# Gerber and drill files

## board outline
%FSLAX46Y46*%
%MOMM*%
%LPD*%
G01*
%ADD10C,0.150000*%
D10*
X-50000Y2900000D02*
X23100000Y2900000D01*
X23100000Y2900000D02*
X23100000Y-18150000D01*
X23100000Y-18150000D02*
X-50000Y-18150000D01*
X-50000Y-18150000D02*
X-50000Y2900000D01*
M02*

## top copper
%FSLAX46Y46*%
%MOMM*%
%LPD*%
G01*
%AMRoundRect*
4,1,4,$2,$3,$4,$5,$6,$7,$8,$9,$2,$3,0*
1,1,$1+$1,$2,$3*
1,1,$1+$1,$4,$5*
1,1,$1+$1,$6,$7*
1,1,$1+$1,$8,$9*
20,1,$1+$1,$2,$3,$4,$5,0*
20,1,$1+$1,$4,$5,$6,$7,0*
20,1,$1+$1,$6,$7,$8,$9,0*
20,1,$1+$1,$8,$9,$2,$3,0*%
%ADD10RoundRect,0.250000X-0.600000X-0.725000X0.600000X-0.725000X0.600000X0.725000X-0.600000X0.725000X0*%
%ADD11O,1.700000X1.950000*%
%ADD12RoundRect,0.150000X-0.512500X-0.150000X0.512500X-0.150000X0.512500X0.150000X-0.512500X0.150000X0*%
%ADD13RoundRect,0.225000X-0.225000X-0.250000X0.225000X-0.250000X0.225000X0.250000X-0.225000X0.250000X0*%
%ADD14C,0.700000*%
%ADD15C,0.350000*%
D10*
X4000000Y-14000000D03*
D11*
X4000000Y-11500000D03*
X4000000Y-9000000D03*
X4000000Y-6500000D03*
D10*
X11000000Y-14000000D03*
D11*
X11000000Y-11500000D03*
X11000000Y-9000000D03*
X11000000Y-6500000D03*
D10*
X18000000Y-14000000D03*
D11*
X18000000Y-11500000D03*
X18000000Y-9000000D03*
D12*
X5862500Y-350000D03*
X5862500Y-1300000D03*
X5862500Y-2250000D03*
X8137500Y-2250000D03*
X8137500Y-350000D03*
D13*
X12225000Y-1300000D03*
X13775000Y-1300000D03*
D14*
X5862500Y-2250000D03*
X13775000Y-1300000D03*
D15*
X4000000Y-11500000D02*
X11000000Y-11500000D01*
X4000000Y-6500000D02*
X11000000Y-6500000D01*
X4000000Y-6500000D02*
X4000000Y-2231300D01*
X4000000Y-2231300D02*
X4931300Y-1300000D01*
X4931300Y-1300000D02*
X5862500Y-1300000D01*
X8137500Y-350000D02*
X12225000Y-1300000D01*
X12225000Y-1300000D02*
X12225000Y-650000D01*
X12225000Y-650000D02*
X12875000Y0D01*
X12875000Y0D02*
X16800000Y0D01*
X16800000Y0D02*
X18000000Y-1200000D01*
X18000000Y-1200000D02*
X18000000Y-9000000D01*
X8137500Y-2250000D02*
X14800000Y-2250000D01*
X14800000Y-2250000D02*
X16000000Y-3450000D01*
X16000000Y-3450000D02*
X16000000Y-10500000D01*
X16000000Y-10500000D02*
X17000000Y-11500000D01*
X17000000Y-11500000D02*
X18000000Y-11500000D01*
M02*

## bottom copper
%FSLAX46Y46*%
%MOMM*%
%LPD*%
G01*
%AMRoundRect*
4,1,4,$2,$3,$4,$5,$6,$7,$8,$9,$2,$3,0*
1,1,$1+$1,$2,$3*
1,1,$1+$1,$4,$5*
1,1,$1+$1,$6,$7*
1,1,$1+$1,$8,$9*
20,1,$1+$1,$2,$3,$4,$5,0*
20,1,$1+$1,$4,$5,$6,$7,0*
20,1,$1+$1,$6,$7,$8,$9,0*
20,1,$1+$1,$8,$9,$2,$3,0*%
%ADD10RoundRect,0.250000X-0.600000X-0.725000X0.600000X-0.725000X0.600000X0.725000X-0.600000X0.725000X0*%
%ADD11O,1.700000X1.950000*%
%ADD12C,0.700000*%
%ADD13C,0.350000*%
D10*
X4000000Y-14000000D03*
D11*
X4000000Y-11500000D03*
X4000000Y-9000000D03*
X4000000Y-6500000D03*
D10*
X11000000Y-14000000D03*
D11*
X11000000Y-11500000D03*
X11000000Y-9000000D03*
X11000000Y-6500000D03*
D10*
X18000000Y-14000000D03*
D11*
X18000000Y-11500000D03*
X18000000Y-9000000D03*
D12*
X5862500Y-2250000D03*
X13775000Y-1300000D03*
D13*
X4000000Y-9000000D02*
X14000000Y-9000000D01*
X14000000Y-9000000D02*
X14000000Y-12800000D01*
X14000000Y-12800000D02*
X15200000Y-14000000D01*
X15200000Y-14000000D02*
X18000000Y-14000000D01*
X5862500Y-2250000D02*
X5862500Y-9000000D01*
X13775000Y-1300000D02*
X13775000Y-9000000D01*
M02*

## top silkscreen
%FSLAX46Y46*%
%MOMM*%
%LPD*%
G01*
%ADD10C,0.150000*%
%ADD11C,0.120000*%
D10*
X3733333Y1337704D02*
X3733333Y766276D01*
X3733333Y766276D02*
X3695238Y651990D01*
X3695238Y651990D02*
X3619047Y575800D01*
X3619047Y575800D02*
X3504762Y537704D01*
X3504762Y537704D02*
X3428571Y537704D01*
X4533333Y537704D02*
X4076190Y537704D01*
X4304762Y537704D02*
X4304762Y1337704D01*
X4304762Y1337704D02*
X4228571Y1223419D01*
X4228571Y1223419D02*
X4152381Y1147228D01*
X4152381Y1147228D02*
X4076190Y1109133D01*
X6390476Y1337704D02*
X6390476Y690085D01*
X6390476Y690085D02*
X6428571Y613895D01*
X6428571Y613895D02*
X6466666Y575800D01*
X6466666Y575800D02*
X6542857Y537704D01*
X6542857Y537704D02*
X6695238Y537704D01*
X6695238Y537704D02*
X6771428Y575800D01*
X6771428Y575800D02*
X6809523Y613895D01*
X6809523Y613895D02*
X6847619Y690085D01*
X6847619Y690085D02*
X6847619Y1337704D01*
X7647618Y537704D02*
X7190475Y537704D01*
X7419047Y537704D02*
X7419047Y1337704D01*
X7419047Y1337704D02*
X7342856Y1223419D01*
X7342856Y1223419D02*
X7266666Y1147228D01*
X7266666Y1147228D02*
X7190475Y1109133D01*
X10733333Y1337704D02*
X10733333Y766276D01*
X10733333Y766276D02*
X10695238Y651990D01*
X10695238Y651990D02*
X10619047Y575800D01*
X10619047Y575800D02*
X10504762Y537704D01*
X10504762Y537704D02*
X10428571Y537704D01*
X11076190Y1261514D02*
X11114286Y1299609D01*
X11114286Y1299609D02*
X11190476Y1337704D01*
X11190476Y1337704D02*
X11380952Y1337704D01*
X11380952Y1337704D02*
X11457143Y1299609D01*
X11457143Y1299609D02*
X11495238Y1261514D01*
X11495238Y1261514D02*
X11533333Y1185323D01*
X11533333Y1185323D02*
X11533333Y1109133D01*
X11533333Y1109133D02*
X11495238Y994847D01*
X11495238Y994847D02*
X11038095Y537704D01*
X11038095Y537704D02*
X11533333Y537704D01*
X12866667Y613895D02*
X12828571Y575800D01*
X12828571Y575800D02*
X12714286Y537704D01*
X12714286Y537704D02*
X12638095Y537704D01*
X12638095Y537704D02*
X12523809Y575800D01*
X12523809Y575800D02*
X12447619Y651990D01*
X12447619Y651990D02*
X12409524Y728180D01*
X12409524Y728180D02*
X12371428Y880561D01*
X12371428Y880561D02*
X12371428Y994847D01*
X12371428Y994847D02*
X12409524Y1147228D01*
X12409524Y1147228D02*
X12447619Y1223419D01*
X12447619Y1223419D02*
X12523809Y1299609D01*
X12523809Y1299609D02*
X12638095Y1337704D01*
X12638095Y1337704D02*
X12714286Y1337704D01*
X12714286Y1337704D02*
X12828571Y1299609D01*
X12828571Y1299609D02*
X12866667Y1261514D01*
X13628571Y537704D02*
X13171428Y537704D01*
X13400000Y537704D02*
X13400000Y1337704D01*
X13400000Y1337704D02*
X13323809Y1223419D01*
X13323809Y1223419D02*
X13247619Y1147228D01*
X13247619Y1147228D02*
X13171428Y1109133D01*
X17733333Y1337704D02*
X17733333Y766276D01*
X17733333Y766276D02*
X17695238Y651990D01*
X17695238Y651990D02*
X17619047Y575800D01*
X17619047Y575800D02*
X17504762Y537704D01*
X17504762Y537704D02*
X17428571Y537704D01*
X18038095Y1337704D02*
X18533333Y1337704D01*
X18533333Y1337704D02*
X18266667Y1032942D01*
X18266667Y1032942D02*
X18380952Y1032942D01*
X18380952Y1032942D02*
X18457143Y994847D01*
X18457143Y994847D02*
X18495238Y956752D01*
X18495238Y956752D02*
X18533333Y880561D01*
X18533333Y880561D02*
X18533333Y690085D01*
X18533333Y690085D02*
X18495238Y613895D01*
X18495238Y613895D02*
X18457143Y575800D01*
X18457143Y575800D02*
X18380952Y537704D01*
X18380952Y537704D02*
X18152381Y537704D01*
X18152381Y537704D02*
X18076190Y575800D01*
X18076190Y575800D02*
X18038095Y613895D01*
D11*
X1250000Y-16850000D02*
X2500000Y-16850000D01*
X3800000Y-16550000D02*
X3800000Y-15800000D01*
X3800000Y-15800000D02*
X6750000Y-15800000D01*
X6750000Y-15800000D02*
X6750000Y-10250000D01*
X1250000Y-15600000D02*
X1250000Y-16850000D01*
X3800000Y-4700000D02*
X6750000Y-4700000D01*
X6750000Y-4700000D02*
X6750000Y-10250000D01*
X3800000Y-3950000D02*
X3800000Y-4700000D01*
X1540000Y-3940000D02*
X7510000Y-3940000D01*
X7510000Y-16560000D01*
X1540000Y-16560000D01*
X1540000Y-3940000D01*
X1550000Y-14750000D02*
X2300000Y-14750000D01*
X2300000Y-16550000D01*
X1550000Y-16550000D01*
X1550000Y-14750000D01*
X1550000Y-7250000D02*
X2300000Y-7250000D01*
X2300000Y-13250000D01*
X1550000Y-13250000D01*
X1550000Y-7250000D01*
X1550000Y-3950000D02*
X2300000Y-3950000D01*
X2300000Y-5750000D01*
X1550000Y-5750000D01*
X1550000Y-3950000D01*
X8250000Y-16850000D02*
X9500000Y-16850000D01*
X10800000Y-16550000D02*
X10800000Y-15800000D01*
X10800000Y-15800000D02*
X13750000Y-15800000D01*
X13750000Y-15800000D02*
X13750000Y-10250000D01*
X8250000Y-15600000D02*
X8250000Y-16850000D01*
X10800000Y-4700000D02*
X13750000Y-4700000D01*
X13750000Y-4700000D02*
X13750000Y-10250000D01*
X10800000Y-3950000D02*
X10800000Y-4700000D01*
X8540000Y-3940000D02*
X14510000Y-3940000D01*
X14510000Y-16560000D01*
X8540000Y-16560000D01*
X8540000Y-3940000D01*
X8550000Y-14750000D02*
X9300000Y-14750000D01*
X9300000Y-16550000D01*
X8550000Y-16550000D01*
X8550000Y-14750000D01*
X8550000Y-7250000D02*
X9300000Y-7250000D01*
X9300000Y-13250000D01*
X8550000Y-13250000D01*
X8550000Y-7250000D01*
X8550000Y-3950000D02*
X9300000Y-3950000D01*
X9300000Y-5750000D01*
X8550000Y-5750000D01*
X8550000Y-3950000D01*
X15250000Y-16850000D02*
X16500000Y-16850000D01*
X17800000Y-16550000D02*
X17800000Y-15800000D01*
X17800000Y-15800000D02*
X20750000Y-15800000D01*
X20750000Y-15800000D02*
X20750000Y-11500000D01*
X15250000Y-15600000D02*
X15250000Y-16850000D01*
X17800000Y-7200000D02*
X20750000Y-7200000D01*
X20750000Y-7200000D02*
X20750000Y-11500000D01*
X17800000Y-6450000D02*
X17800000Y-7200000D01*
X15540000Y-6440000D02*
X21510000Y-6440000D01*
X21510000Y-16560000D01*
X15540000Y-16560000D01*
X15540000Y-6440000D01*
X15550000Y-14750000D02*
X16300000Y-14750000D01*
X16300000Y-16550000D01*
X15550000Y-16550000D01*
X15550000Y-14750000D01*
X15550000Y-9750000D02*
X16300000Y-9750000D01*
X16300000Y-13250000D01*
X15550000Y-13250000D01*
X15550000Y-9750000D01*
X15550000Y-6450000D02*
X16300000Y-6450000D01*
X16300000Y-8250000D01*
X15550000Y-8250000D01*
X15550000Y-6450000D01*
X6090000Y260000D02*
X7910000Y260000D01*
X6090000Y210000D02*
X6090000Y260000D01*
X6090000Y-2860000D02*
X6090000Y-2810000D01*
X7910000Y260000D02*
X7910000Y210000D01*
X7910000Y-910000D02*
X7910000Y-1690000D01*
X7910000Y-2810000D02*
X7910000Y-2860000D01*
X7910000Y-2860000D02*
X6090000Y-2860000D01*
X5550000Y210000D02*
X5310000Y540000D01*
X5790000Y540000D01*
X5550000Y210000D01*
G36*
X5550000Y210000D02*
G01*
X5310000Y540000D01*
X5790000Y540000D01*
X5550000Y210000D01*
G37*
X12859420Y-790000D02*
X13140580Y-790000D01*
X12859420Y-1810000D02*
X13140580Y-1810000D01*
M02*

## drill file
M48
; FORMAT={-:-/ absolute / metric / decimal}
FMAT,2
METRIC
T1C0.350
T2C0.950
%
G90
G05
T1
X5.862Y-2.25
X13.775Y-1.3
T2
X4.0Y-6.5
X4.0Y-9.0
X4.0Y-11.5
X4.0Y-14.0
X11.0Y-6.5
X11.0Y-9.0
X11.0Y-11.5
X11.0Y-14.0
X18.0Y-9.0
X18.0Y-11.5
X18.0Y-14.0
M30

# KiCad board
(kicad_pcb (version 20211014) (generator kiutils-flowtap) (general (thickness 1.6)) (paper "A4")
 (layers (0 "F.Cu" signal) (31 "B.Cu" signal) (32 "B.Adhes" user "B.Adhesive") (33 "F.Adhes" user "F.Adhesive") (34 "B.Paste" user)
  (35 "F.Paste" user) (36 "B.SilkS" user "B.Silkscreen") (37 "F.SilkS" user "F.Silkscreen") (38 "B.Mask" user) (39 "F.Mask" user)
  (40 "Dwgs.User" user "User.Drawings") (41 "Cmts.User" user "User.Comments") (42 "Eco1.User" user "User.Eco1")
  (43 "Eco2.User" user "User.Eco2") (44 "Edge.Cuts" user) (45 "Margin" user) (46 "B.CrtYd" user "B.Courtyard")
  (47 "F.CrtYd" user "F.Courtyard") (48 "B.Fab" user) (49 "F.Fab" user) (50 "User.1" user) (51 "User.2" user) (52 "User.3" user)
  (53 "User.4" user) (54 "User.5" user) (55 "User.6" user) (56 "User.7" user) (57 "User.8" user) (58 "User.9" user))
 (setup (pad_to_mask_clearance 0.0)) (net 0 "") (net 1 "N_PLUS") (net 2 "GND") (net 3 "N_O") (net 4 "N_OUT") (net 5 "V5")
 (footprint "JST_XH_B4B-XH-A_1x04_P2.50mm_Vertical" (layer "F.Cu") (at 4 14 90) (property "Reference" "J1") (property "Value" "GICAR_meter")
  (fp_line (start -2.85 -2.75) (end -2.85 -1.5) (layer "F.SilkS") (stroke (width 0.12) (type solid)))
  (fp_line (start -2.55 -0.2) (end -1.8 -0.2) (layer "F.SilkS") (stroke (width 0.12) (type solid)))
  (fp_line (start -1.8 -0.2) (end -1.8 2.75) (layer "F.SilkS") (stroke (width 0.12) (type solid)))
  (fp_line (start -1.8 2.75) (end 3.75 2.75) (layer "F.SilkS") (stroke (width 0.12) (type solid)))
  (fp_line (start -1.6 -2.75) (end -2.85 -2.75) (layer "F.SilkS") (stroke (width 0.12) (type solid)))
  (fp_line (start 9.3 -0.2) (end 9.3 2.75) (layer "F.SilkS") (stroke (width 0.12) (type solid)))
  (fp_line (start 9.3 2.75) (end 3.75 2.75) (layer "F.SilkS") (stroke (width 0.12) (type solid)))
  (fp_line (start 10.05 -0.2) (end 9.3 -0.2) (layer "F.SilkS") (stroke (width 0.12) (type solid)))
  (fp_rect (start -2.56 -2.46) (end 10.06 3.51) (layer "F.SilkS") (stroke (width 0.12) (type solid)) (fill no))
  (fp_rect (start -2.55 -2.45) (end -0.75 -1.7) (layer "F.SilkS") (stroke (width 0.12) (type solid)) (fill no))
  (fp_rect (start 0.75 -2.45) (end 6.75 -1.7) (layer "F.SilkS") (stroke (width 0.12) (type solid)) (fill no))
  (fp_rect (start 8.25 -2.45) (end 10.05 -1.7) (layer "F.SilkS") (stroke (width 0.12) (type solid)) (fill no))
  (pad "1" thru_hole roundrect (at 0 0) (size 1.7 1.95) (drill 0.95) (layers *.Cu *.Mask) (remove_unused_layers no)
   (roundrect_rratio 0.147059))
  (pad "2" thru_hole oval (at 2.5 0) (size 1.7 1.95) (drill 0.95) (layers *.Cu *.Mask) (remove_unused_layers no) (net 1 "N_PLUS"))
  (pad "3" thru_hole oval (at 5 0) (size 1.7 1.95) (drill 0.95) (layers *.Cu *.Mask) (remove_unused_layers no) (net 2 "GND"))
  (pad "4" thru_hole oval (at 7.5 0) (size 1.7 1.95) (drill 0.95) (layers *.Cu *.Mask) (remove_unused_layers no) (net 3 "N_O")))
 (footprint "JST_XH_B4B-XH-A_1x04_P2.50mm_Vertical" (layer "F.Cu") (at 11 14 90) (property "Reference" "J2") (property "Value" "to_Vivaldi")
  (fp_line (start -2.85 -2.75) (end -2.85 -1.5) (layer "F.SilkS") (stroke (width 0.12) (type solid)))
  (fp_line (start -2.55 -0.2) (end -1.8 -0.2) (layer "F.SilkS") (stroke (width 0.12) (type solid)))
  (fp_line (start -1.8 -0.2) (end -1.8 2.75) (layer "F.SilkS") (stroke (width 0.12) (type solid)))
  (fp_line (start -1.8 2.75) (end 3.75 2.75) (layer "F.SilkS") (stroke (width 0.12) (type solid)))
  (fp_line (start -1.6 -2.75) (end -2.85 -2.75) (layer "F.SilkS") (stroke (width 0.12) (type solid)))
  (fp_line (start 9.3 -0.2) (end 9.3 2.75) (layer "F.SilkS") (stroke (width 0.12) (type solid)))
  (fp_line (start 9.3 2.75) (end 3.75 2.75) (layer "F.SilkS") (stroke (width 0.12) (type solid)))
  (fp_line (start 10.05 -0.2) (end 9.3 -0.2) (layer "F.SilkS") (stroke (width 0.12) (type solid)))
  (fp_rect (start -2.56 -2.46) (end 10.06 3.51) (layer "F.SilkS") (stroke (width 0.12) (type solid)) (fill no))
  (fp_rect (start -2.55 -2.45) (end -0.75 -1.7) (layer "F.SilkS") (stroke (width 0.12) (type solid)) (fill no))
  (fp_rect (start 0.75 -2.45) (end 6.75 -1.7) (layer "F.SilkS") (stroke (width 0.12) (type solid)) (fill no))
  (fp_rect (start 8.25 -2.45) (end 10.05 -1.7) (layer "F.SilkS") (stroke (width 0.12) (type solid)) (fill no))
  (pad "1" thru_hole roundrect (at 0 0) (size 1.7 1.95) (drill 0.95) (layers *.Cu *.Mask) (remove_unused_layers no)
   (roundrect_rratio 0.147059))
  (pad "2" thru_hole oval (at 2.5 0) (size 1.7 1.95) (drill 0.95) (layers *.Cu *.Mask) (remove_unused_layers no) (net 1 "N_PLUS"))
  (pad "3" thru_hole oval (at 5 0) (size 1.7 1.95) (drill 0.95) (layers *.Cu *.Mask) (remove_unused_layers no) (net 2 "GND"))
  (pad "4" thru_hole oval (at 7.5 0) (size 1.7 1.95) (drill 0.95) (layers *.Cu *.Mask) (remove_unused_layers no) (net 3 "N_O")))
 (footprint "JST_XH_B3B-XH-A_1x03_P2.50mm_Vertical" (layer "F.Cu") (at 18 14 90) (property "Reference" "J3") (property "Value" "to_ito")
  (fp_line (start -2.85 -2.75) (end -2.85 -1.5) (layer "F.SilkS") (stroke (width 0.12) (type solid)))
  (fp_line (start -2.55 -0.2) (end -1.8 -0.2) (layer "F.SilkS") (stroke (width 0.12) (type solid)))
  (fp_line (start -1.8 -0.2) (end -1.8 2.75) (layer "F.SilkS") (stroke (width 0.12) (type solid)))
  (fp_line (start -1.8 2.75) (end 2.5 2.75) (layer "F.SilkS") (stroke (width 0.12) (type solid)))
  (fp_line (start -1.6 -2.75) (end -2.85 -2.75) (layer "F.SilkS") (stroke (width 0.12) (type solid)))
  (fp_line (start 6.8 -0.2) (end 6.8 2.75) (layer "F.SilkS") (stroke (width 0.12) (type solid)))
  (fp_line (start 6.8 2.75) (end 2.5 2.75) (layer "F.SilkS") (stroke (width 0.12) (type solid)))
  (fp_line (start 7.55 -0.2) (end 6.8 -0.2) (layer "F.SilkS") (stroke (width 0.12) (type solid)))
  (fp_rect (start -2.56 -2.46) (end 7.56 3.51) (layer "F.SilkS") (stroke (width 0.12) (type solid)) (fill no))
  (fp_rect (start -2.55 -2.45) (end -0.75 -1.7) (layer "F.SilkS") (stroke (width 0.12) (type solid)) (fill no))
  (fp_rect (start 0.75 -2.45) (end 4.25 -1.7) (layer "F.SilkS") (stroke (width 0.12) (type solid)) (fill no))
  (fp_rect (start 5.75 -2.45) (end 7.55 -1.7) (layer "F.SilkS") (stroke (width 0.12) (type solid)) (fill no))
  (pad "1" thru_hole roundrect (at 0 0) (size 1.7 1.95) (drill 0.95) (layers *.Cu *.Mask) (remove_unused_layers no)
   (roundrect_rratio 0.147059) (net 2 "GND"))
  (pad "2" thru_hole oval (at 2.5 0) (size 1.7 1.95) (drill 0.95) (layers *.Cu *.Mask) (remove_unused_layers no) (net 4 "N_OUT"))
  (pad "3" thru_hole oval (at 5 0) (size 1.7 1.95) (drill 0.95) (layers *.Cu *.Mask) (remove_unused_layers no) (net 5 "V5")))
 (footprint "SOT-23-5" (layer "F.Cu") (at 7 1.3) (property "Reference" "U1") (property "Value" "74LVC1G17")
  (fp_line (start -0.91 -1.56) (end 0.91 -1.56) (layer "F.SilkS") (stroke (width 0.12) (type solid)))
  (fp_line (start -0.91 -1.51) (end -0.91 -1.56) (layer "F.SilkS") (stroke (width 0.12) (type solid)))
  (fp_line (start -0.91 1.56) (end -0.91 1.51) (layer "F.SilkS") (stroke (width 0.12) (type solid)))
  (fp_line (start 0.91 -1.56) (end 0.91 -1.51) (layer "F.SilkS") (stroke (width 0.12) (type solid)))
  (fp_line (start 0.91 -0.39) (end 0.91 0.39) (layer "F.SilkS") (stroke (width 0.12) (type solid)))
  (fp_line (start 0.91 1.51) (end 0.91 1.56) (layer "F.SilkS") (stroke (width 0.12) (type solid)))
  (fp_line (start 0.91 1.56) (end -0.91 1.56) (layer "F.SilkS") (stroke (width 0.12) (type solid)))
  (fp_poly (pts (xy -1.45 -1.51) (xy -1.69 -1.84) (xy -1.21 -1.84)) (layer "F.SilkS") (stroke (width 0.12) (type solid)) (fill yes))
  (pad "1" smd roundrect (at -1.1375 -0.95) (size 1.325 0.6) (layers "F.Cu" "F.Mask" "F.Paste") (roundrect_rratio 0.25))
  (pad "2" smd roundrect (at -1.1375 0) (size 1.325 0.6) (layers "F.Cu" "F.Mask" "F.Paste") (roundrect_rratio 0.25) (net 3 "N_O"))
  (pad "3" smd roundrect (at -1.1375 0.95) (size 1.325 0.6) (layers "F.Cu" "F.Mask" "F.Paste") (roundrect_rratio 0.25) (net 2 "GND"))
  (pad "4" smd roundrect (at 1.1375 0.95) (size 1.325 0.6) (layers "F.Cu" "F.Mask" "F.Paste") (roundrect_rratio 0.25) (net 4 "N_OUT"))
  (pad "5" smd roundrect (at 1.1375 -0.95) (size 1.325 0.6) (layers "F.Cu" "F.Mask" "F.Paste") (roundrect_rratio 0.25) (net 5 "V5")))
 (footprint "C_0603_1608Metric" (layer "F.Cu") (at 13 1.3) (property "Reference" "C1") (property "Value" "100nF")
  (fp_line (start -0.14058 -0.51) (end 0.14058 -0.51) (layer "F.SilkS") (stroke (width 0.12) (type solid)))
  (fp_line (start -0.14058 0.51) (end 0.14058 0.51) (layer "F.SilkS") (stroke (width 0.12) (type solid)))
  (pad "1" smd roundrect (at -0.775 0) (size 0.9 0.95) (layers "F.Cu" "F.Mask" "F.Paste") (roundrect_rratio 0.25) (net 5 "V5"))
  (pad "2" smd roundrect (at 0.775 0) (size 0.9 0.95) (layers "F.Cu" "F.Mask" "F.Paste") (roundrect_rratio 0.25) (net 2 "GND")))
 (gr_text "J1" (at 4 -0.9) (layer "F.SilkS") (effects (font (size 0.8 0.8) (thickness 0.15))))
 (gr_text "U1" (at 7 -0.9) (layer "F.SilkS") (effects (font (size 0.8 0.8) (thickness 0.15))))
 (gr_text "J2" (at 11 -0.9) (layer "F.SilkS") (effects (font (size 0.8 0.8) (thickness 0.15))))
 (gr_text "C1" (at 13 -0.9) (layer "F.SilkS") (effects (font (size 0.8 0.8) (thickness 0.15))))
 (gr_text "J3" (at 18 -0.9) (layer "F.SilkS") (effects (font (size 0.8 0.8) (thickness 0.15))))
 (gr_line (start -0.05 -2.9) (end 23.1 -2.9) (layer "Edge.Cuts") (width 0.15))
 (gr_line (start 23.1 -2.9) (end 23.1 18.15) (layer "Edge.Cuts") (width 0.15))
 (gr_line (start 23.1 18.15) (end -0.05 18.15) (layer "Edge.Cuts") (width 0.15))
 (gr_line (start -0.05 18.15) (end -0.05 -2.9) (layer "Edge.Cuts") (width 0.15))
 (segment (start 4.0 11.5) (end 11.0 11.5) (width 0.35) (layer "F.Cu") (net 1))
 (segment (start 4.0 6.5) (end 11.0 6.5) (width 0.35) (layer "F.Cu") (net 3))
 (segment (start 4.0 6.5) (end 4.0 2.2313) (width 0.35) (layer "F.Cu") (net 3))
 (segment (start 4.0 2.2313) (end 4.9313 1.3) (width 0.35) (layer "F.Cu") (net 3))
 (segment (start 4.9313 1.3) (end 5.8625 1.3) (width 0.35) (layer "F.Cu") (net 3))
 (segment (start 8.1375 0.35) (end 12.225 1.3) (width 0.35) (layer "F.Cu") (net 5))
 (segment (start 12.225 1.3) (end 12.225 0.65) (width 0.35) (layer "F.Cu") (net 5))
 (segment (start 12.225 0.65) (end 12.875 0.0) (width 0.35) (layer "F.Cu") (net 5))
 (segment (start 12.875 0.0) (end 16.8 0.0) (width 0.35) (layer "F.Cu") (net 5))
 (segment (start 16.8 0.0) (end 18.0 1.2) (width 0.35) (layer "F.Cu") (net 5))
 (segment (start 18.0 1.2) (end 18.0 9.0) (width 0.35) (layer "F.Cu") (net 5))
 (segment (start 8.1375 2.25) (end 14.8 2.25) (width 0.35) (layer "F.Cu") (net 4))
 (segment (start 14.8 2.25) (end 16.0 3.45) (width 0.35) (layer "F.Cu") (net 4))
 (segment (start 16.0 3.45) (end 16.0 10.5) (width 0.35) (layer "F.Cu") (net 4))
 (segment (start 16.0 10.5) (end 17.0 11.5) (width 0.35) (layer "F.Cu") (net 4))
 (segment (start 17.0 11.5) (end 18.0 11.5) (width 0.35) (layer "F.Cu") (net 4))
 (segment (start 4.0 9.0) (end 14.0 9.0) (width 0.35) (layer "B.Cu") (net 2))
 (segment (start 14.0 9.0) (end 14.0 12.8) (width 0.35) (layer "B.Cu") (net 2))
 (segment (start 14.0 12.8) (end 15.2 14.0) (width 0.35) (layer "B.Cu") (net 2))
 (segment (start 15.2 14.0) (end 18.0 14.0) (width 0.35) (layer "B.Cu") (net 2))
 (via (at 5.8625 2.25) (size 0.7) (drill 0.35) (layers "F.Cu" "B.Cu") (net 2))
 (segment (start 5.8625 2.25) (end 5.8625 9.0) (width 0.35) (layer "B.Cu") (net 2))
 (via (at 13.775 1.3) (size 0.7) (drill 0.35) (layers "F.Cu" "B.Cu") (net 2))
 (segment (start 13.775 1.3) (end 13.775 9.0) (width 0.35) (layer "B.Cu") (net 2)))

